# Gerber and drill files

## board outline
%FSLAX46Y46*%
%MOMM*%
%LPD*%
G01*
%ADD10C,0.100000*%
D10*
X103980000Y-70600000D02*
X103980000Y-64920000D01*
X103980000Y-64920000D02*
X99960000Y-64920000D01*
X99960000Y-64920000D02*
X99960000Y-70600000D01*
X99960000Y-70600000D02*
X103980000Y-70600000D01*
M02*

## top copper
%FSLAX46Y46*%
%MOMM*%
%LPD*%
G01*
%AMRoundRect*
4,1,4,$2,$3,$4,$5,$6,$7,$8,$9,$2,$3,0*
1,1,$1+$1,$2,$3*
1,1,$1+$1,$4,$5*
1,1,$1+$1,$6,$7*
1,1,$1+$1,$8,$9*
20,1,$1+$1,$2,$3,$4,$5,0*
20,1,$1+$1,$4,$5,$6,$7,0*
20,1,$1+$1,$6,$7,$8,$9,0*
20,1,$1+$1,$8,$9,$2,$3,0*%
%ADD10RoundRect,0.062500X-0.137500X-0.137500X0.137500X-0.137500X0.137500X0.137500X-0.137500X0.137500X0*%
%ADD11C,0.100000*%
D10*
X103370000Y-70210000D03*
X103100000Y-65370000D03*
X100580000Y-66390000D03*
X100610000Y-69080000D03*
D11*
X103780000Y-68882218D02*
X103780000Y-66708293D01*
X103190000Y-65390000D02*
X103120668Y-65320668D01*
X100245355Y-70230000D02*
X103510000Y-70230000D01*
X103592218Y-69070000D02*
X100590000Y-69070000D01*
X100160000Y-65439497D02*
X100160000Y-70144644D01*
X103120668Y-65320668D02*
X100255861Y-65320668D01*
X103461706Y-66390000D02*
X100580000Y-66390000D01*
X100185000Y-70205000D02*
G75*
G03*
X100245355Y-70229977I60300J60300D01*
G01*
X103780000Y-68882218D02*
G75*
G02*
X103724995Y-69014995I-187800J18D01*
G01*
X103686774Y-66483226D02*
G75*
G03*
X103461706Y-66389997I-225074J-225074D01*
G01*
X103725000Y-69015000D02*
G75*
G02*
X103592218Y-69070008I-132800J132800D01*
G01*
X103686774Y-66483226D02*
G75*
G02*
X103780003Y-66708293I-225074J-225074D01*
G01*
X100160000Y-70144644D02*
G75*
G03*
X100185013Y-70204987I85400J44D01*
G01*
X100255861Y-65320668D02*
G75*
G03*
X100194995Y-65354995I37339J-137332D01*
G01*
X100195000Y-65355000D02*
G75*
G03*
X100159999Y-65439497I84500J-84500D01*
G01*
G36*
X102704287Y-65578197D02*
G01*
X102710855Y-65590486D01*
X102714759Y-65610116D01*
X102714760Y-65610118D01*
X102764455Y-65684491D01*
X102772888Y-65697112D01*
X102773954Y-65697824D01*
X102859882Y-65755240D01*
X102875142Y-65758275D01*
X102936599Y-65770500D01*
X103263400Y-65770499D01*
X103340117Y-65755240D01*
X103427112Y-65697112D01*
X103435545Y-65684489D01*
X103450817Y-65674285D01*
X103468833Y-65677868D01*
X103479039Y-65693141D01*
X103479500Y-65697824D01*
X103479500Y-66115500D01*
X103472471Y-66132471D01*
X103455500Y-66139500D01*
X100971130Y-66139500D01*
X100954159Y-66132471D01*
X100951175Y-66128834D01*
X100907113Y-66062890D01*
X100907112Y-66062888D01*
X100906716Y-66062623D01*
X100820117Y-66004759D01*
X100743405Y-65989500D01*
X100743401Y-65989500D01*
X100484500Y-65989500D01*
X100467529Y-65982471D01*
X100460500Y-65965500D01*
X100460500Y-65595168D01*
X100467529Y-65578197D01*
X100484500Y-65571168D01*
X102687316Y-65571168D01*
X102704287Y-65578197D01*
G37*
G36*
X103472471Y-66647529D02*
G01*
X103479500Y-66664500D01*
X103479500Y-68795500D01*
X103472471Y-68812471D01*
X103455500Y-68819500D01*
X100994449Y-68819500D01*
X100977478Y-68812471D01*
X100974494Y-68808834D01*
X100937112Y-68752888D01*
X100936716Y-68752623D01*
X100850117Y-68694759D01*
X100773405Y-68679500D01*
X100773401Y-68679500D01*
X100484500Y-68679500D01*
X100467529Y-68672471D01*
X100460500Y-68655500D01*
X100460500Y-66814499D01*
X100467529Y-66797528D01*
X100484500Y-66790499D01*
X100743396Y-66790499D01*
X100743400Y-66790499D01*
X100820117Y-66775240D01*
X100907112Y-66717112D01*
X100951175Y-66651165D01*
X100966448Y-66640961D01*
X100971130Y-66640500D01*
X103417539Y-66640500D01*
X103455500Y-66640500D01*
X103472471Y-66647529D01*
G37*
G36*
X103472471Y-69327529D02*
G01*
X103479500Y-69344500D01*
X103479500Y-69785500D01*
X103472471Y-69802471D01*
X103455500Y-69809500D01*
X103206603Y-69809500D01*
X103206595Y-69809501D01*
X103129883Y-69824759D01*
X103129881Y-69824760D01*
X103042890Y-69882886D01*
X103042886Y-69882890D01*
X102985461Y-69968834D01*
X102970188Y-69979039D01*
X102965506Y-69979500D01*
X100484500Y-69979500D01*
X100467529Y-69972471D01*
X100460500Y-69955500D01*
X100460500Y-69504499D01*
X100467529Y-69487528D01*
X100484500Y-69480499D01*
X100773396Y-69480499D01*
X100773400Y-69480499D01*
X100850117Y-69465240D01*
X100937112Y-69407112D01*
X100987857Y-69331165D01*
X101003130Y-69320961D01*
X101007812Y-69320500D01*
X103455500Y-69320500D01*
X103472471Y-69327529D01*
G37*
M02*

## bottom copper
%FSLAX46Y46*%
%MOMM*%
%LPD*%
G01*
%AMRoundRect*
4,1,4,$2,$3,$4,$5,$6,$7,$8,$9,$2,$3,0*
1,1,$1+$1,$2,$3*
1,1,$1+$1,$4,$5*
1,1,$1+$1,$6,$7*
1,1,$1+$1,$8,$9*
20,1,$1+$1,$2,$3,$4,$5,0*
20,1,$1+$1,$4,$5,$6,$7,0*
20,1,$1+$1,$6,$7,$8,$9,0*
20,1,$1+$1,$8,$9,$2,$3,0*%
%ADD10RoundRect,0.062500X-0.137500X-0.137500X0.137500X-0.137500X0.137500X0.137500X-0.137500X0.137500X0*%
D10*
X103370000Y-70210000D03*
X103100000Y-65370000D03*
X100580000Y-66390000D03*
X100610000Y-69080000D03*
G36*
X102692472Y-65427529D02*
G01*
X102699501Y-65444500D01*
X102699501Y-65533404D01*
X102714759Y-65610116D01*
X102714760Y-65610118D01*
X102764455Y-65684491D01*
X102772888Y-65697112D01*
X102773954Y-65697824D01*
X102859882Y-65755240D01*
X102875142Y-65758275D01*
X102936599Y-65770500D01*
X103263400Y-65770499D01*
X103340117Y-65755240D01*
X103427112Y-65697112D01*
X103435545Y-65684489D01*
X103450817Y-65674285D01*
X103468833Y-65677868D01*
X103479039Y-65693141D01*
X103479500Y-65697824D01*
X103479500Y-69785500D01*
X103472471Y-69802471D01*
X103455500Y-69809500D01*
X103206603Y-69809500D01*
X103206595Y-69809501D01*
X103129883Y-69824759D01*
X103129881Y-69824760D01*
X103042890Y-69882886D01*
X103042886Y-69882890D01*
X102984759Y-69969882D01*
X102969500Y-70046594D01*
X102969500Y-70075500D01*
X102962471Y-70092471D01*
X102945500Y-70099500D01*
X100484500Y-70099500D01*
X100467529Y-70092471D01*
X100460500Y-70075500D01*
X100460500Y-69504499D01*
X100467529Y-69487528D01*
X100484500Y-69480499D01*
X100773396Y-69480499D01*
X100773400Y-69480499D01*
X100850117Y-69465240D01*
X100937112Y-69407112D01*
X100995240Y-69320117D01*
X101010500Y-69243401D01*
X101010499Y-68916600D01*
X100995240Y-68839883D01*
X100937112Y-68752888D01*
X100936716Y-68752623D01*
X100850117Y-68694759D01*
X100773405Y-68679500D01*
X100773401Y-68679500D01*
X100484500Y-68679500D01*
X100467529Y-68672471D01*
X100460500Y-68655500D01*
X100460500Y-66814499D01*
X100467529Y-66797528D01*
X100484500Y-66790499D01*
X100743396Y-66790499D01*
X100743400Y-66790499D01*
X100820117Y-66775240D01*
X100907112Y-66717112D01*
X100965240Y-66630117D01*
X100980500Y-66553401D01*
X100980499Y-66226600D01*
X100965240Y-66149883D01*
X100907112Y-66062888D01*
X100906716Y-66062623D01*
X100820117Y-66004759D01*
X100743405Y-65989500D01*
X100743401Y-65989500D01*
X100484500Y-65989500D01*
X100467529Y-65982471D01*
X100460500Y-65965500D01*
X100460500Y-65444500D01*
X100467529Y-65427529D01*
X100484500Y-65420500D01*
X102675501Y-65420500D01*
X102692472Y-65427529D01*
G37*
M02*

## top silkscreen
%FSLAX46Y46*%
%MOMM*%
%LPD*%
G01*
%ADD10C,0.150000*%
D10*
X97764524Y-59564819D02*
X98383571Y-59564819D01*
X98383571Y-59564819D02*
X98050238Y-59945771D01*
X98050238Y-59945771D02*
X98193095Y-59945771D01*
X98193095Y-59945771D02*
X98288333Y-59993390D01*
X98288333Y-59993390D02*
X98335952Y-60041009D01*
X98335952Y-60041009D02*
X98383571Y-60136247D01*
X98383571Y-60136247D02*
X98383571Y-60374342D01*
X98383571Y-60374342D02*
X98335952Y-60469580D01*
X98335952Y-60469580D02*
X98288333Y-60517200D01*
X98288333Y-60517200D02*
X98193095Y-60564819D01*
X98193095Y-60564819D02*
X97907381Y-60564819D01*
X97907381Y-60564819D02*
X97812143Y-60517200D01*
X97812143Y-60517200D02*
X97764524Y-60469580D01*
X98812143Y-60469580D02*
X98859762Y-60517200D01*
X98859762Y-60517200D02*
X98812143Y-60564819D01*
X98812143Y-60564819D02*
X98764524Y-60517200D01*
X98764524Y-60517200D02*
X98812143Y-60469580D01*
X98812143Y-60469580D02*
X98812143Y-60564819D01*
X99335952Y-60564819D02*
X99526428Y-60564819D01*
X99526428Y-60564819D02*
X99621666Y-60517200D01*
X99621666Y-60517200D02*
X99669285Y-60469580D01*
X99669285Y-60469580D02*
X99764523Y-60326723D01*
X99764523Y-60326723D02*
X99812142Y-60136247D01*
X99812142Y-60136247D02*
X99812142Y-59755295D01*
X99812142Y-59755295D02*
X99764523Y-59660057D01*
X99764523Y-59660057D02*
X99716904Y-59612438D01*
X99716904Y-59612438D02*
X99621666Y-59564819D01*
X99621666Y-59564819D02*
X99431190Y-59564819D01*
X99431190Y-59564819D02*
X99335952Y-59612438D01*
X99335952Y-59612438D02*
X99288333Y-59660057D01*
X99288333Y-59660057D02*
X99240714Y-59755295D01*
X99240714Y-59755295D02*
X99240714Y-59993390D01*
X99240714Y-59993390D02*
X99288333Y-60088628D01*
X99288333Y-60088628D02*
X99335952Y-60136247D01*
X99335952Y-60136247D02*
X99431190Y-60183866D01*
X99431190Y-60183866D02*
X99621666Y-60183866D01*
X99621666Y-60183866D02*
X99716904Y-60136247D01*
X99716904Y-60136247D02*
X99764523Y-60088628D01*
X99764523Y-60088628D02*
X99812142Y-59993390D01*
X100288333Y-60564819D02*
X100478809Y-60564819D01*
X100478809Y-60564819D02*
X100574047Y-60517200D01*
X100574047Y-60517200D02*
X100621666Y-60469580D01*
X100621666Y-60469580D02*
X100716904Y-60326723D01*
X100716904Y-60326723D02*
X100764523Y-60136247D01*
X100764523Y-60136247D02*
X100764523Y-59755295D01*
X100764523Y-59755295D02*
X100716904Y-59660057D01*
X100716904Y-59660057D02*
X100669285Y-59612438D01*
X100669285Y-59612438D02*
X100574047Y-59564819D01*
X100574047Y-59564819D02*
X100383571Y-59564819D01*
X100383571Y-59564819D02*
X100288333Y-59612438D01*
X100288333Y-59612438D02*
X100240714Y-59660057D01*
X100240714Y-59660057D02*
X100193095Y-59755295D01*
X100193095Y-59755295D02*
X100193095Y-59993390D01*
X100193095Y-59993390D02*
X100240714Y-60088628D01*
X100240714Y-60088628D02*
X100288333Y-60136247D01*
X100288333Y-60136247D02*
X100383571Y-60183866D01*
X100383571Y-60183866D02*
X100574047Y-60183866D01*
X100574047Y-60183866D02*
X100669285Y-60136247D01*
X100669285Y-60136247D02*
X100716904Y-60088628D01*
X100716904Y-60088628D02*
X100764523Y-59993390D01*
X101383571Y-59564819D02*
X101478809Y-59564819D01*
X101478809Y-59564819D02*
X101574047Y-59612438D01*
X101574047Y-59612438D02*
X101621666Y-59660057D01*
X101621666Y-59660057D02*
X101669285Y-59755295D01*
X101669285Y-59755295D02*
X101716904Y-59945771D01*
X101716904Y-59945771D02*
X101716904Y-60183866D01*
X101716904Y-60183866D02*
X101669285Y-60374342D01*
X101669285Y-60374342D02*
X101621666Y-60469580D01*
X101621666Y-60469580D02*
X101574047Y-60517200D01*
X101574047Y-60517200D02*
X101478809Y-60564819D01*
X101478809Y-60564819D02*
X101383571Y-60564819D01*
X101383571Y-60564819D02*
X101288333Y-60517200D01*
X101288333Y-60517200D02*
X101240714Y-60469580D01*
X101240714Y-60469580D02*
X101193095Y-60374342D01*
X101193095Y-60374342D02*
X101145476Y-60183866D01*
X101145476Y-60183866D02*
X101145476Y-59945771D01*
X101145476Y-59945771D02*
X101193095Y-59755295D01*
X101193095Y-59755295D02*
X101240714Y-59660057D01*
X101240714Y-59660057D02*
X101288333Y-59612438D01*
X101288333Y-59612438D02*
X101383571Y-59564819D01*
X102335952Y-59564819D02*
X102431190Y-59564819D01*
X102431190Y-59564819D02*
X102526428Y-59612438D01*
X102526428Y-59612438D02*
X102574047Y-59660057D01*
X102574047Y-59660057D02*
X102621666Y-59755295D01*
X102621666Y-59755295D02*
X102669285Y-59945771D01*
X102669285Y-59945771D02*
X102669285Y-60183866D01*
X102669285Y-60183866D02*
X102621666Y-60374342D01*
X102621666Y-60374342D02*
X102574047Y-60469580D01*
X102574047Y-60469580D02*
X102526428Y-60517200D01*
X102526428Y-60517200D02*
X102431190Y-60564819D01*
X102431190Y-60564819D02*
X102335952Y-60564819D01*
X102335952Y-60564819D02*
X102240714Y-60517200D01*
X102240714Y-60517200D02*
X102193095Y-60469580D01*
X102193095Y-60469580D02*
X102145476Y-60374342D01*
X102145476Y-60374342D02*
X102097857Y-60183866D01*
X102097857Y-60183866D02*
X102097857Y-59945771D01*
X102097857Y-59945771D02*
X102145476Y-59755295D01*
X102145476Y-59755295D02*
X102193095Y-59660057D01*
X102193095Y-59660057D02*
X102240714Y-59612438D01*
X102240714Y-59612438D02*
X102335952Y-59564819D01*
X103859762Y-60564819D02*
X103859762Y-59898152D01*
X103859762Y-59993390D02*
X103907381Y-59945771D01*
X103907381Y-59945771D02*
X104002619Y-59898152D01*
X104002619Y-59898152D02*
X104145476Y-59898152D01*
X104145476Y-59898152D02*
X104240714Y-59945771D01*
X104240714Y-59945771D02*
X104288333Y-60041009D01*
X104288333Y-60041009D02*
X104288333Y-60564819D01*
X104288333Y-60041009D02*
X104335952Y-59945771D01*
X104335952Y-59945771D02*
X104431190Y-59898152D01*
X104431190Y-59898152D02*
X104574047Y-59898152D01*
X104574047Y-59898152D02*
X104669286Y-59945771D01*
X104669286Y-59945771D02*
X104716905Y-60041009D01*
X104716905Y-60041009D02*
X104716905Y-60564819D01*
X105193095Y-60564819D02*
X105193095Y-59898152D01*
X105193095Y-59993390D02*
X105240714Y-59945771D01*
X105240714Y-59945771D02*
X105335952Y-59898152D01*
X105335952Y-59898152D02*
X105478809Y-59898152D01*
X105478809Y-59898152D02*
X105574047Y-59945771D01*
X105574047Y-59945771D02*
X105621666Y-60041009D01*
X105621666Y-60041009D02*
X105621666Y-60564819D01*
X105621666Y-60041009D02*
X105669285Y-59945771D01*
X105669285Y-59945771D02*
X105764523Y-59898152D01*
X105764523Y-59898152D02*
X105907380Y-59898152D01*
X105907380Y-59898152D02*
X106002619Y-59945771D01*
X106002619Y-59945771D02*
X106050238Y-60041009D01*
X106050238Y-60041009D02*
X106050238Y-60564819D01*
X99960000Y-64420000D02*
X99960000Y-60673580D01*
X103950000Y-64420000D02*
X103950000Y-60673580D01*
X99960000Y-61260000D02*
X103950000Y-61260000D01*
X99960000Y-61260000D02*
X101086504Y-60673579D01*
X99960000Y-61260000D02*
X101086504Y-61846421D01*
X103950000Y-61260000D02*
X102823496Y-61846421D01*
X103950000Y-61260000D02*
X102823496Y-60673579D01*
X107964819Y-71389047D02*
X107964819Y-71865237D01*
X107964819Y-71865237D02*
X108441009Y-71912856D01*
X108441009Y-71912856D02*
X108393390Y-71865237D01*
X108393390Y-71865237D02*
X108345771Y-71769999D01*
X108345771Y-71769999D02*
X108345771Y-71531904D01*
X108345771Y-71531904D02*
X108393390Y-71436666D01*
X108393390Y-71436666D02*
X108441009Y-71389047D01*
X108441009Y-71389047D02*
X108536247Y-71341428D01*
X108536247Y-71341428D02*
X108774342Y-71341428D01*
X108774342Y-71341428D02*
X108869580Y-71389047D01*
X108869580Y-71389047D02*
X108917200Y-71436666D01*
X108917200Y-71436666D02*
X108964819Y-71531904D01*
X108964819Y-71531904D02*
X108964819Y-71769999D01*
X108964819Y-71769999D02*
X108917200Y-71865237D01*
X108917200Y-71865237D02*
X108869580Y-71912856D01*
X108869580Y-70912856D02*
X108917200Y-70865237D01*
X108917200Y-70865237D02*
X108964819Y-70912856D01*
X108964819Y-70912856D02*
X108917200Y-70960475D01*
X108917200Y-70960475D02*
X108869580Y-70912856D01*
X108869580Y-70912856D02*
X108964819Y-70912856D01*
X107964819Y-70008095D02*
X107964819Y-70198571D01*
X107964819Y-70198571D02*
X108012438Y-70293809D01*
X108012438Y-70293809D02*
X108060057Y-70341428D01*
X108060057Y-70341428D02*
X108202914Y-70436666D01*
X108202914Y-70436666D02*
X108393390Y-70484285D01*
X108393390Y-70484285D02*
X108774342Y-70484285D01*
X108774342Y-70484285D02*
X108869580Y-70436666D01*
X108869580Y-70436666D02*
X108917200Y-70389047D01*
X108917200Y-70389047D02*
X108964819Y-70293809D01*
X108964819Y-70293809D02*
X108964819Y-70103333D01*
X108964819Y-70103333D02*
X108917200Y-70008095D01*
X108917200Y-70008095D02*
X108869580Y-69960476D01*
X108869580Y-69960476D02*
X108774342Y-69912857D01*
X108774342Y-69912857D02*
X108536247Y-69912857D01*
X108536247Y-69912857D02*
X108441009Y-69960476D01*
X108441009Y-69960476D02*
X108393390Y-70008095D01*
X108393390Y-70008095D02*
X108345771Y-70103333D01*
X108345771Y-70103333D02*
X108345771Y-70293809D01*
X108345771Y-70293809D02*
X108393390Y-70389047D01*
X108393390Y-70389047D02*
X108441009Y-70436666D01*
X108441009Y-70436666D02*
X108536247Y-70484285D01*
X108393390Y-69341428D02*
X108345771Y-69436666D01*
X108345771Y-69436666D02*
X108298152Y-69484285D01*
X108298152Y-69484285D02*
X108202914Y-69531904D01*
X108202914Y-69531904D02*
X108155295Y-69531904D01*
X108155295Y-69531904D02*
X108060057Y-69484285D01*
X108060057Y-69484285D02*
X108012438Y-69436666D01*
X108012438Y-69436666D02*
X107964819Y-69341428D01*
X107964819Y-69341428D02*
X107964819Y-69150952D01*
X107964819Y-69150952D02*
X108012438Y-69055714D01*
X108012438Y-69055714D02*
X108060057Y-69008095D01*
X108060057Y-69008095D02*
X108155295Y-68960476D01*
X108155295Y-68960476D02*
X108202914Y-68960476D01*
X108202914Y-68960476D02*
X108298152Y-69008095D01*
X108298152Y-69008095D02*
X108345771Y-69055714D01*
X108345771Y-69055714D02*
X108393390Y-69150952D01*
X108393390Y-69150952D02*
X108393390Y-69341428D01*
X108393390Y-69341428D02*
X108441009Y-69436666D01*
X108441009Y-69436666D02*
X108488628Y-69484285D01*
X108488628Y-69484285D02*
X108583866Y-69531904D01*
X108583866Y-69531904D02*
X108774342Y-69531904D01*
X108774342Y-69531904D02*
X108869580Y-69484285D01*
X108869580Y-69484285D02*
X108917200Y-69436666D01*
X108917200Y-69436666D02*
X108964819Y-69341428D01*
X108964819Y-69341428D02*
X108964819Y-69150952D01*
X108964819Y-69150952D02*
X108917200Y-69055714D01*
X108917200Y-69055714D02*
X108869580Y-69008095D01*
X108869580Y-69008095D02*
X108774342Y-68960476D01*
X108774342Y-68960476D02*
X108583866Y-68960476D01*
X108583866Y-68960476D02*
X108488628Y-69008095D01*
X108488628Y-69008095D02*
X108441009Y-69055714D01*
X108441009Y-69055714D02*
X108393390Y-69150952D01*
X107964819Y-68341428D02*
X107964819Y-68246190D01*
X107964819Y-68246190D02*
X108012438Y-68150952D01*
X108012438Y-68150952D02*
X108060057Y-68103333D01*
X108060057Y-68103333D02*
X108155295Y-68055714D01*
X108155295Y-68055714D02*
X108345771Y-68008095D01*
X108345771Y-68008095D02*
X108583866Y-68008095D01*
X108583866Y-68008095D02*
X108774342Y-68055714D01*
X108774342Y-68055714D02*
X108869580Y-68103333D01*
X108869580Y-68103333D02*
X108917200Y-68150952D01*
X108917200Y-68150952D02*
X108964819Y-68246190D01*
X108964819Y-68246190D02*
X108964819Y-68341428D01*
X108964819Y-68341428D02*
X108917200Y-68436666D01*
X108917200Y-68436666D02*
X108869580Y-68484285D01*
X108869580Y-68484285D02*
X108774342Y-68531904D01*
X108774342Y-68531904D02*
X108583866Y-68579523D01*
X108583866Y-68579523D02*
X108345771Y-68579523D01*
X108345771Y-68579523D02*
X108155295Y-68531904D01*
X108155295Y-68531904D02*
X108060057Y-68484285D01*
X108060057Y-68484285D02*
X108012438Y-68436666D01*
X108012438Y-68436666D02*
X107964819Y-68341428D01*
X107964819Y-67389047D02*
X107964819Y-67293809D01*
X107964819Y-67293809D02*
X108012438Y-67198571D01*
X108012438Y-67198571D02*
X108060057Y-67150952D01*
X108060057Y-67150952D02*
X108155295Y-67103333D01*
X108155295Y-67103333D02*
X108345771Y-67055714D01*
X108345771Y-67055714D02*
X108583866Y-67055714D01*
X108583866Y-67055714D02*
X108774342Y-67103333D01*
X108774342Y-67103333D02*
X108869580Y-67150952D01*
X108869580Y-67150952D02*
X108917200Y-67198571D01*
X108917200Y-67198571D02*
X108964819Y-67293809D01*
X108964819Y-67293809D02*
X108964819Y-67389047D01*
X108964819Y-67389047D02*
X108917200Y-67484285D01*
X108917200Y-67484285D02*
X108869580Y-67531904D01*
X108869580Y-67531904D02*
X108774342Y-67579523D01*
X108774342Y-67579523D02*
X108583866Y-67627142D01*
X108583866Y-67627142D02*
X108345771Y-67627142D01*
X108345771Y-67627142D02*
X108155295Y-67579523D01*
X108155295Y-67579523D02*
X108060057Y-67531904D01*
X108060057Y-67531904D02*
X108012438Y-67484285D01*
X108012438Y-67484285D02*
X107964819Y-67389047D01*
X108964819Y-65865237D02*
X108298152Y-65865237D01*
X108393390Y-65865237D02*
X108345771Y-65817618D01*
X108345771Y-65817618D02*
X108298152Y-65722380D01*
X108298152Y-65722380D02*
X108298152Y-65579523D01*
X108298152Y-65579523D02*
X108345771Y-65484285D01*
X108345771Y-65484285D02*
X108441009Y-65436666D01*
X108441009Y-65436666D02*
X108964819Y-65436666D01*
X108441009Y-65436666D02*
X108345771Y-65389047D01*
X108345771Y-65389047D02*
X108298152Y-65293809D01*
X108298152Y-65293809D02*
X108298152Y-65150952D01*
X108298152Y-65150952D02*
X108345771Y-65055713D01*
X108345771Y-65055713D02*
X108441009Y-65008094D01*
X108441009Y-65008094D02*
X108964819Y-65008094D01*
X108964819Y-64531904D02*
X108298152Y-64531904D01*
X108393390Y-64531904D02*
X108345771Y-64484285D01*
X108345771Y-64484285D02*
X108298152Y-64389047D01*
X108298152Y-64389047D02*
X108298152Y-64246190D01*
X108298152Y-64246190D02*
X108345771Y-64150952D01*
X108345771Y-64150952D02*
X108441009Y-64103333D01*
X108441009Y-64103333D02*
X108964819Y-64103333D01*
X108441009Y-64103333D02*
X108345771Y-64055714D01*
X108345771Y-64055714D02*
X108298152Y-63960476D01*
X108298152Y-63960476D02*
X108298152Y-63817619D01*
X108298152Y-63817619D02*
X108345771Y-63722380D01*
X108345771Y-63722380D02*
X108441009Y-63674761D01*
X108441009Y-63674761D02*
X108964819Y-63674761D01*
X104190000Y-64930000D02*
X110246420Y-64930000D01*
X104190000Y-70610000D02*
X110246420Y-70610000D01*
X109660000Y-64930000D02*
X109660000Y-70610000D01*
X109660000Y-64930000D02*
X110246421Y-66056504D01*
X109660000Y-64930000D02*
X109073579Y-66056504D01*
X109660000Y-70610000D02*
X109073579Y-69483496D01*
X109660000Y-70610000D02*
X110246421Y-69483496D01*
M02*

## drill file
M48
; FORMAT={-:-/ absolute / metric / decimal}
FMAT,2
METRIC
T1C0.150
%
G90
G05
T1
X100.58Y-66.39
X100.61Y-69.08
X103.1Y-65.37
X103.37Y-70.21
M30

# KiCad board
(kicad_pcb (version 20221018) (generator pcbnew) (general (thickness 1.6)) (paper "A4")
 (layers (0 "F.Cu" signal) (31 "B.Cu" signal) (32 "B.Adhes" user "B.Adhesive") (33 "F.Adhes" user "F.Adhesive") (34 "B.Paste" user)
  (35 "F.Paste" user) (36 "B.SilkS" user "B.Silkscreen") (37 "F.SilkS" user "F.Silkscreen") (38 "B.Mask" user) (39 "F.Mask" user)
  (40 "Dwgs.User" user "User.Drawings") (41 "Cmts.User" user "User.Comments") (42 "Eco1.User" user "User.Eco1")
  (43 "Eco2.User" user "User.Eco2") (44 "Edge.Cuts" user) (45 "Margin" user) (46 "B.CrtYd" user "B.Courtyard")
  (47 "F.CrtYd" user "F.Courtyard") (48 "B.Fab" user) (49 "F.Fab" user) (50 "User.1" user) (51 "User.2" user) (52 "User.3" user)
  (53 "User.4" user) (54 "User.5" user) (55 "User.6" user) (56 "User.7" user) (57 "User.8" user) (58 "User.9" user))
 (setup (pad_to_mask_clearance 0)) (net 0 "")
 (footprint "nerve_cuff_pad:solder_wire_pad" (layer "F.Cu") (at 103.37 70.21)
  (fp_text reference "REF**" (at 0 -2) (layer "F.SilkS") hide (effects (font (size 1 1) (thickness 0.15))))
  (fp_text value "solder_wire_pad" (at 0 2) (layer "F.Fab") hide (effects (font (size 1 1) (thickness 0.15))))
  (pad "1" thru_hole roundrect (at 0 0) (size 0.4 0.4) (drill 0.15) (layers "*.Cu" "*.Mask") (roundrect_rratio 0.15625)))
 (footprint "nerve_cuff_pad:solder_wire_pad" (layer "F.Cu") (at 103.1 65.37)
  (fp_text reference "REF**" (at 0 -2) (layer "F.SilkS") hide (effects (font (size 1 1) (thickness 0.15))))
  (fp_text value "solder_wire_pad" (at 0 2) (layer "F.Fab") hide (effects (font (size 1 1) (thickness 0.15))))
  (pad "1" thru_hole roundrect (at 0 0) (size 0.4 0.4) (drill 0.15) (layers "*.Cu" "*.Mask") (roundrect_rratio 0.15625)))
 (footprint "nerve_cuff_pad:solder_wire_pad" (layer "F.Cu") (at 100.58 66.39)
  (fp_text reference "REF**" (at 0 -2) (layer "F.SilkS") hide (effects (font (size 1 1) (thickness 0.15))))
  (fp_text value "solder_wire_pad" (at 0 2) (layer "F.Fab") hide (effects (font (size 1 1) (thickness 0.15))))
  (pad "1" thru_hole roundrect (at 0 0) (size 0.4 0.4) (drill 0.15) (layers "*.Cu" "*.Mask") (roundrect_rratio 0.15625)))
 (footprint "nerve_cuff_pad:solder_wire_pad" (layer "F.Cu") (at 100.61 69.08)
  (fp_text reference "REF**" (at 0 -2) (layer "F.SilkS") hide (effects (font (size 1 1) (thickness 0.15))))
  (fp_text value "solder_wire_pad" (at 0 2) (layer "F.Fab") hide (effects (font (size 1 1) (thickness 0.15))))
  (pad "1" thru_hole roundrect (at 0 0) (size 0.4 0.4) (drill 0.15) (layers "*.Cu" "*.Mask") (roundrect_rratio 0.15625)))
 (gr_line (start 103.98 70.6) (end 103.98 64.92) (stroke (width 0.1) (type default)) (layer "Edge.Cuts"))
 (gr_line (start 103.98 64.92) (end 99.96 64.92) (stroke (width 0.1) (type default)) (layer "Edge.Cuts"))
 (gr_line (start 99.96 64.92) (end 99.96 70.6) (stroke (width 0.1) (type default)) (layer "Edge.Cuts"))
 (gr_line (start 99.96 70.6) (end 103.98 70.6) (stroke (width 0.1) (type default)) (layer "Edge.Cuts"))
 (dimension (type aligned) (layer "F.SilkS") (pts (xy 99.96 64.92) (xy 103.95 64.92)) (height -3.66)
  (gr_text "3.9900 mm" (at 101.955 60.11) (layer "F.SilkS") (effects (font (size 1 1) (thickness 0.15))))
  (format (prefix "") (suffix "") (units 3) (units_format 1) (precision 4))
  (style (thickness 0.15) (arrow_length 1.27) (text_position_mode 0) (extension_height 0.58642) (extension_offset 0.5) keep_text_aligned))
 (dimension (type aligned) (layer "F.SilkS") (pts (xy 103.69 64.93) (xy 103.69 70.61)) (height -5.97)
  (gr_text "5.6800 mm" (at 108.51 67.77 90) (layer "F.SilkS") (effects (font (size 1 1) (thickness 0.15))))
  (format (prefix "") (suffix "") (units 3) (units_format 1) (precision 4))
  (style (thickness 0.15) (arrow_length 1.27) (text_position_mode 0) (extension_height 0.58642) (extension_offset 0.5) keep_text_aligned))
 (segment (start 103.78 68.882218) (end 103.78 66.708293) (width 0.1) (layer "F.Cu") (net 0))
 (segment (start 103.19 65.39) (end 103.120668 65.320668) (width 0.1) (layer "F.Cu") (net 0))
 (segment (start 100.245355 70.23) (end 103.51 70.23) (width 0.1) (layer "F.Cu") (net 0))
 (segment (start 103.592218 69.07) (end 100.59 69.07) (width 0.1) (layer "F.Cu") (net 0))
 (segment (start 100.16 65.439497) (end 100.16 70.144644) (width 0.1) (layer "F.Cu") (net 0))
 (segment (start 103.120668 65.320668) (end 100.255861 65.320668) (width 0.1) (layer "F.Cu") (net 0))
 (segment (start 103.461706 66.39) (end 100.58 66.39) (width 0.1) (layer "F.Cu") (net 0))
 (arc (start 100.185 70.205) (mid 100.212691 70.223508) (end 100.245355 70.23) (width 0.1) (layer "F.Cu") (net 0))
 (arc (start 103.78 68.882218) (mid 103.765705 68.954079) (end 103.725 69.015) (width 0.1) (layer "F.Cu") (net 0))
 (arc (start 103.686774 66.483226) (mid 103.583512 66.414228) (end 103.461706 66.39) (width 0.1) (layer "F.Cu") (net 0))
 (arc (start 103.725 69.015) (mid 103.664079 69.055705) (end 103.592218 69.07) (width 0.1) (layer "F.Cu") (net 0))
 (arc (start 103.686774 66.483226) (mid 103.755771 66.586487) (end 103.78 66.708293) (width 0.1) (layer "F.Cu") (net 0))
 (arc (start 100.16 70.144644) (mid 100.166497 70.177308) (end 100.185 70.205) (width 0.1) (layer "F.Cu") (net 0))
 (arc (start 100.255861 65.320668) (mid 100.223167 65.33411) (end 100.195 65.355) (width 0.1) (layer "F.Cu") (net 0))
 (arc (start 100.195 65.355) (mid 100.169096 65.393767) (end 100.16 65.439497) (width 0.1) (layer "F.Cu") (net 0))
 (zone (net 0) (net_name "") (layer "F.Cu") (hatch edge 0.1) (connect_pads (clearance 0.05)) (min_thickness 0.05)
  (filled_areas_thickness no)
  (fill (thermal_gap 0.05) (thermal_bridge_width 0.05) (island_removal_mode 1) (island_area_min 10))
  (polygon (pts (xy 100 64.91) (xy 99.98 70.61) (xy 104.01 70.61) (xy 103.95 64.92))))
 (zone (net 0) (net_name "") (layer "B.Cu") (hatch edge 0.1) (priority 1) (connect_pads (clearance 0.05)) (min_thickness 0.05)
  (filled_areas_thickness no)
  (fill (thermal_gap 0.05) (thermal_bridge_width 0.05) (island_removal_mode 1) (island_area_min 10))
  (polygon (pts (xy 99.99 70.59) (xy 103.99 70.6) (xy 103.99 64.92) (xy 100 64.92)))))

